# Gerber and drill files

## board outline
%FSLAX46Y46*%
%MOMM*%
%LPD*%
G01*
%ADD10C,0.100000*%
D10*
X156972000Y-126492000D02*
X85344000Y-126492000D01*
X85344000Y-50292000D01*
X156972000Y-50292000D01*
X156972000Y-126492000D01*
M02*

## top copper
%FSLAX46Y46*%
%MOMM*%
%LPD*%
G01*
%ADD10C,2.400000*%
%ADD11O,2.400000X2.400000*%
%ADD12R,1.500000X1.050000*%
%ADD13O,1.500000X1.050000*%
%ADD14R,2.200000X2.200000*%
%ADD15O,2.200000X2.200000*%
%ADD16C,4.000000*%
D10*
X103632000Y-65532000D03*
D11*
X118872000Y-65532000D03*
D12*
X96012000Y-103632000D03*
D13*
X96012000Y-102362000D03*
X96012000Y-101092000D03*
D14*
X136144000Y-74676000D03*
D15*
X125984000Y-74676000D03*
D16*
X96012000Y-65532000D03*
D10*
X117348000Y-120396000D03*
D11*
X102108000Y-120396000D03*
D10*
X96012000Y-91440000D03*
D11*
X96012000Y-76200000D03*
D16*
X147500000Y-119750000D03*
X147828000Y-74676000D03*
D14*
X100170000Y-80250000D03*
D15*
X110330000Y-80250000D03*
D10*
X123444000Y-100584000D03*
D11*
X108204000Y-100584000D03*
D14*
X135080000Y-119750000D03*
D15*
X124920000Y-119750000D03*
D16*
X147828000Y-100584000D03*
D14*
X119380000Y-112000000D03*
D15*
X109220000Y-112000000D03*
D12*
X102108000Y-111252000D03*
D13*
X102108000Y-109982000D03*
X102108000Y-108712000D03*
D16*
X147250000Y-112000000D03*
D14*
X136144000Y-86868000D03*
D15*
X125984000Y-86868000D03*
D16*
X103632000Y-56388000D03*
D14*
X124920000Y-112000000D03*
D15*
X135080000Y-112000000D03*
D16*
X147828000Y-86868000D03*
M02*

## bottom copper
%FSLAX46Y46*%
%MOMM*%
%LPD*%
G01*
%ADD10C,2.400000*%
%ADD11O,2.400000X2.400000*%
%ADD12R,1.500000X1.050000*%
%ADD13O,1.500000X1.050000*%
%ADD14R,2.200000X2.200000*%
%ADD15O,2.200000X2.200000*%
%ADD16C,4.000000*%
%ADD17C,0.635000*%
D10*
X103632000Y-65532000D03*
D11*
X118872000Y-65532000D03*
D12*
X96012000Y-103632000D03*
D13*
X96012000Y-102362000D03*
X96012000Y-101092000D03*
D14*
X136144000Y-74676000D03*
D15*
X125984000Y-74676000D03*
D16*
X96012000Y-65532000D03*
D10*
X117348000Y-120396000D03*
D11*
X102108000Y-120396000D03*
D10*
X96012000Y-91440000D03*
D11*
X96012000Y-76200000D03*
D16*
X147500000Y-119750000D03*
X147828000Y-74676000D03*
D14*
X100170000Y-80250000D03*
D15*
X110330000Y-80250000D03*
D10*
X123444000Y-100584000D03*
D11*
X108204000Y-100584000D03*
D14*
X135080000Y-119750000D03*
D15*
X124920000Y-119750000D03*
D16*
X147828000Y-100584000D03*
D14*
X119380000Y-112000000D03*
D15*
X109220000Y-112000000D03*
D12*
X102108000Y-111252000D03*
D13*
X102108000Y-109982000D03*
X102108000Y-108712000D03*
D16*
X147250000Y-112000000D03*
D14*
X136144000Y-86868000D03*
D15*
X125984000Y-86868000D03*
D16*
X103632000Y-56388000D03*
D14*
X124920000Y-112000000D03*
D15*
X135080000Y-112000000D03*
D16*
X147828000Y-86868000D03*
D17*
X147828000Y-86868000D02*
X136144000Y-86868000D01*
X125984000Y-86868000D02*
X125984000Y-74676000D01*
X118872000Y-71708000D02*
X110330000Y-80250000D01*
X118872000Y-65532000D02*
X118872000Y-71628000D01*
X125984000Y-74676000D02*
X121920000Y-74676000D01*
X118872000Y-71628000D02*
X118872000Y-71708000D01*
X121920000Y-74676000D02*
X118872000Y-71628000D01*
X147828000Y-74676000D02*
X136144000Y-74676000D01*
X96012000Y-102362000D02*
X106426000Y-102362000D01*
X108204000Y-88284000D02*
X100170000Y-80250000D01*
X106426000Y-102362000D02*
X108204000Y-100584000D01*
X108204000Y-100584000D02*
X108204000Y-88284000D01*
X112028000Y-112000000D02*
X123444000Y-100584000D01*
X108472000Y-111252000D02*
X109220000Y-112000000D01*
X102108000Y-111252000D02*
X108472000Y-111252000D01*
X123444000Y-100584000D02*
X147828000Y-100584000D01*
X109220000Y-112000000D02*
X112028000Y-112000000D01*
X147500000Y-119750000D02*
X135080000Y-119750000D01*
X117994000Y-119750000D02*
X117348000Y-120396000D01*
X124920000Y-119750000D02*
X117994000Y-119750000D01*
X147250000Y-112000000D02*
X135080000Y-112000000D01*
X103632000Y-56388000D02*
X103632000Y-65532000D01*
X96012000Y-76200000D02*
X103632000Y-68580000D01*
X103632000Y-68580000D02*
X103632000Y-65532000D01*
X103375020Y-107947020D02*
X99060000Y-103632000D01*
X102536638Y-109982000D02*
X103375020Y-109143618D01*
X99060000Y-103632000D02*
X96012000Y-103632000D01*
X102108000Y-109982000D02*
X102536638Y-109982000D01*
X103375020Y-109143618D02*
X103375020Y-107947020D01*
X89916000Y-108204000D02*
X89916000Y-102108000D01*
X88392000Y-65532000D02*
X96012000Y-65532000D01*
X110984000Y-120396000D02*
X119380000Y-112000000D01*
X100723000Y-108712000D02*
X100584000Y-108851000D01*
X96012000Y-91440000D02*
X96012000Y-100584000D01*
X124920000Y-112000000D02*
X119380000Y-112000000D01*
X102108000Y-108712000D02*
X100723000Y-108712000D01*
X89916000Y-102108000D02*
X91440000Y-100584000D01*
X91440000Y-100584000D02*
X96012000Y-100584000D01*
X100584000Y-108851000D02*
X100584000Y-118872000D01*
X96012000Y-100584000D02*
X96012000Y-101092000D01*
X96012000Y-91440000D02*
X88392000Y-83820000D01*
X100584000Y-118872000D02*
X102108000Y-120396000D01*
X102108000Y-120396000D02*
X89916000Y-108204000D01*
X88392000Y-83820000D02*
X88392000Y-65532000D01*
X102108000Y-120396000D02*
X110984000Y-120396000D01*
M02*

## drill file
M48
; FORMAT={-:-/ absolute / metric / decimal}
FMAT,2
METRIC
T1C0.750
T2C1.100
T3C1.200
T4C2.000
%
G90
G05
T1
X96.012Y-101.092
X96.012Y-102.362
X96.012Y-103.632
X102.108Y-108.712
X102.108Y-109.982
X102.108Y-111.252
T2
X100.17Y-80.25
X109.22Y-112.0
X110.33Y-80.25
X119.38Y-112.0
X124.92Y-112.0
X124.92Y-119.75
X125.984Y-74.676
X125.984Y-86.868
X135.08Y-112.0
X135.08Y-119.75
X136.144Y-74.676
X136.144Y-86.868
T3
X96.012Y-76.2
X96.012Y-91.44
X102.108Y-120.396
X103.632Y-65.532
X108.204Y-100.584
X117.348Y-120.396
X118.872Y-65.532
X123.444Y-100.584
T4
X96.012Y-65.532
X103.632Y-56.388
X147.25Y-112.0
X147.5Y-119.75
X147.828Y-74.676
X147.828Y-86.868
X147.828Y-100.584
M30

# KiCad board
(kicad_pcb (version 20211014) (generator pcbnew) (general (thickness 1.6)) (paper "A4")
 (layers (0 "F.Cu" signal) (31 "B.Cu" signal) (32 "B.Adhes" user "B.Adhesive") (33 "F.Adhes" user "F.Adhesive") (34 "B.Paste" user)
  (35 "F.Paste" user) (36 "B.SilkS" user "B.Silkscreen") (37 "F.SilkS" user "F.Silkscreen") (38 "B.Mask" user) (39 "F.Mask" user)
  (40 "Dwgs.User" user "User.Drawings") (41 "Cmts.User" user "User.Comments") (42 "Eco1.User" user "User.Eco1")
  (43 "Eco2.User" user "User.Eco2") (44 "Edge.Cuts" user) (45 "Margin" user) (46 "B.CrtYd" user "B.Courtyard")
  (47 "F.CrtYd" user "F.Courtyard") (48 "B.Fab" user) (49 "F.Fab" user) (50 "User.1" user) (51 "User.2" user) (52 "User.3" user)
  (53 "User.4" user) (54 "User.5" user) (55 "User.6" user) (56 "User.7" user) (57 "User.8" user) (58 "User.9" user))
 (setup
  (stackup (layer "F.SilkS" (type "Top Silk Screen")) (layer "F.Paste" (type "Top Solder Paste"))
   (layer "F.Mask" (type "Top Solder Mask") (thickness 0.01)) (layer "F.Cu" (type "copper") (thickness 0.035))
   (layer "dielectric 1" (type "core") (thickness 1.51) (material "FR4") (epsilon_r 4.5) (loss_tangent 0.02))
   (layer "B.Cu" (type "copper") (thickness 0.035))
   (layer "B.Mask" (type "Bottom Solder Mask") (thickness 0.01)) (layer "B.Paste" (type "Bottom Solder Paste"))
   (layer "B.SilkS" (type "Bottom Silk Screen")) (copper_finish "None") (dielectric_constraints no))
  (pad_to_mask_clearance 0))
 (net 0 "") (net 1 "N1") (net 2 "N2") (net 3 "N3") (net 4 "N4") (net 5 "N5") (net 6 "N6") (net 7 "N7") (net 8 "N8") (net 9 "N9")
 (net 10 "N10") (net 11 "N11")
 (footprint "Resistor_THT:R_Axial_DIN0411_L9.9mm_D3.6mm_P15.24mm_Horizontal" (layer "F.Cu") (at 103.632 65.532)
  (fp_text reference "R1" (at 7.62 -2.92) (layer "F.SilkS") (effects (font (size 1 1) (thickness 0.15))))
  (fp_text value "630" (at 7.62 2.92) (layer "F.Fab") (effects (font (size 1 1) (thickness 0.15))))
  (pad "1" thru_hole circle (at 0 0) (size 2.4 2.4) (drill 1.2) (layers *.Cu *.Mask) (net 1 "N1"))
  (pad "2" thru_hole oval (at 15.24 0) (size 2.4 2.4) (drill 1.2) (layers *.Cu *.Mask) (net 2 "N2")))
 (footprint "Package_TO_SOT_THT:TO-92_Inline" (layer "F.Cu") (at 96.012 103.632 90)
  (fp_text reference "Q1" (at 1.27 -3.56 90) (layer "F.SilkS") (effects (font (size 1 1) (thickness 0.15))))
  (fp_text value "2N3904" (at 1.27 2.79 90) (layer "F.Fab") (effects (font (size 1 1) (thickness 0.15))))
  (pad "1" thru_hole rect (at 0 0 90) (size 1.05 1.5) (drill 0.75) (layers *.Cu *.Mask) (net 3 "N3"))
  (pad "2" thru_hole oval (at 1.27 0 90) (size 1.05 1.5) (drill 0.75) (layers *.Cu *.Mask) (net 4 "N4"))
  (pad "3" thru_hole oval (at 2.54 0 90) (size 1.05 1.5) (drill 0.75) (layers *.Cu *.Mask) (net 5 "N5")))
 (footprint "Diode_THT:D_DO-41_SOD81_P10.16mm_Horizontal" (layer "F.Cu") (at 136.144 74.676 180)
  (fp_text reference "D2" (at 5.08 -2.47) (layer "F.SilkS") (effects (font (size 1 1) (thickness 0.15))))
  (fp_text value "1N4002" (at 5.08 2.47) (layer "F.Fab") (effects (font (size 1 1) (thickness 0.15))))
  (pad "1" thru_hole rect (at 0 0 180) (size 2.2 2.2) (drill 1.1) (layers *.Cu *.Mask) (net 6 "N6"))
  (pad "2" thru_hole oval (at 10.16 0 180) (size 2.2 2.2) (drill 1.1) (layers *.Cu *.Mask) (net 2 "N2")))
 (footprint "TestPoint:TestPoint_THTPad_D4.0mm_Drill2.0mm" (layer "F.Cu") (at 96.012 65.532)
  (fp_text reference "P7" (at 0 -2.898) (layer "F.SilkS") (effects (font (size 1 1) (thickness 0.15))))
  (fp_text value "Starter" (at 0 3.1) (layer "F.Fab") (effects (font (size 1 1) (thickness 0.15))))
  (pad "1" thru_hole circle (at 0 0) (size 4 4) (drill 2) (layers *.Cu *.Mask) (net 5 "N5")))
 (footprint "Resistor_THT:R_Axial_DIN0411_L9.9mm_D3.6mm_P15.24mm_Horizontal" (layer "F.Cu") (at 117.348 120.396 180)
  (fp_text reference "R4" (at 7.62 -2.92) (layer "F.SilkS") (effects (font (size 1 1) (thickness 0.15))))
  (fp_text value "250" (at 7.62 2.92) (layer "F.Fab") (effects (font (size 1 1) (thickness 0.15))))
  (pad "1" thru_hole circle (at 0 0 180) (size 2.4 2.4) (drill 1.2) (layers *.Cu *.Mask) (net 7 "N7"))
  (pad "2" thru_hole oval (at 15.24 0 180) (size 2.4 2.4) (drill 1.2) (layers *.Cu *.Mask) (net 5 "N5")))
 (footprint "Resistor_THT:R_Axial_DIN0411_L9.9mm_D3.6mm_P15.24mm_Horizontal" (layer "F.Cu") (at 96.012 91.44 90)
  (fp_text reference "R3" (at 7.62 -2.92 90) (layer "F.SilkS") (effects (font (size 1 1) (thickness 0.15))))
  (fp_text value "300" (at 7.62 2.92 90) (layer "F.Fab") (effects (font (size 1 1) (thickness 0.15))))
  (pad "1" thru_hole circle (at 0 0 90) (size 2.4 2.4) (drill 1.2) (layers *.Cu *.Mask) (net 5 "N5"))
  (pad "2" thru_hole oval (at 15.24 0 90) (size 2.4 2.4) (drill 1.2) (layers *.Cu *.Mask) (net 1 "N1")))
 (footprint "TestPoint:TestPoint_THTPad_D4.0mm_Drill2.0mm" (layer "F.Cu") (at 147.5 119.75)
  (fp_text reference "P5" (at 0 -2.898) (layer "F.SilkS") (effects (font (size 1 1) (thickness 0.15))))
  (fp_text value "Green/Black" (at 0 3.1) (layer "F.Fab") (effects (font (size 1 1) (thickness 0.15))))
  (pad "1" thru_hole circle (at 0 0) (size 4 4) (drill 2) (layers *.Cu *.Mask) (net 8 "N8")))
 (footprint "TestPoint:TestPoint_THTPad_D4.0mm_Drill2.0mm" (layer "F.Cu") (at 147.828 74.676)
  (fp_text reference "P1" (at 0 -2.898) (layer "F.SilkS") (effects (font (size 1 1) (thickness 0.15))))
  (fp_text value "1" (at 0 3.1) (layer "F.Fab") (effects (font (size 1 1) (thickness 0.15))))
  (pad "1" thru_hole circle (at 0 0) (size 4 4) (drill 2) (layers *.Cu *.Mask) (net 6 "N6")))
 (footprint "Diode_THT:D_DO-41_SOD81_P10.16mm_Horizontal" (layer "F.Cu") (at 100.17 80.25)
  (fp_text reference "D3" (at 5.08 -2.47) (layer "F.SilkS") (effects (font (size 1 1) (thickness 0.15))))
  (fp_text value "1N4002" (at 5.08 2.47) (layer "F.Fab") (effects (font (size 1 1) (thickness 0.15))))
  (pad "1" thru_hole rect (at 0 0) (size 2.2 2.2) (drill 1.1) (layers *.Cu *.Mask) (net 4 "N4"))
  (pad "2" thru_hole oval (at 10.16 0) (size 2.2 2.2) (drill 1.1) (layers *.Cu *.Mask) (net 2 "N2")))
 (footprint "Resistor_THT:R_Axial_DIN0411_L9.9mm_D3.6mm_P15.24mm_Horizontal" (layer "F.Cu") (at 123.444 100.584 180)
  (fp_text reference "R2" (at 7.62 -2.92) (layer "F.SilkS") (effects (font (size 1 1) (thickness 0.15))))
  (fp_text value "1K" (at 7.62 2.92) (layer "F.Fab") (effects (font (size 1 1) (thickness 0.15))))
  (pad "1" thru_hole circle (at 0 0 180) (size 2.4 2.4) (drill 1.2) (layers *.Cu *.Mask) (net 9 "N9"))
  (pad "2" thru_hole oval (at 15.24 0 180) (size 2.4 2.4) (drill 1.2) (layers *.Cu *.Mask) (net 4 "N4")))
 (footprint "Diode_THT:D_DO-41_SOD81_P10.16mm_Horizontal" (layer "F.Cu") (at 135.08 119.75 180)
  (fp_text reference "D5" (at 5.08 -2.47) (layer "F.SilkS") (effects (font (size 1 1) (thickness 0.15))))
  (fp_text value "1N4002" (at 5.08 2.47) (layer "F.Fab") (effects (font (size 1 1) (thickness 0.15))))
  (pad "1" thru_hole rect (at 0 0 180) (size 2.2 2.2) (drill 1.1) (layers *.Cu *.Mask) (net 8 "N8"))
  (pad "2" thru_hole oval (at 10.16 0 180) (size 2.2 2.2) (drill 1.1) (layers *.Cu *.Mask) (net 7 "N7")))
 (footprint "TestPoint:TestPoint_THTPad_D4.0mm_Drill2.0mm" (layer "F.Cu") (at 147.828 100.584)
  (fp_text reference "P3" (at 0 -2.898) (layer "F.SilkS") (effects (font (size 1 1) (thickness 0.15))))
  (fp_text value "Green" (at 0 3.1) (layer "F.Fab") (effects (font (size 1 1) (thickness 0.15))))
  (pad "1" thru_hole circle (at 0 0) (size 4 4) (drill 2) (layers *.Cu *.Mask) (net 9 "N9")))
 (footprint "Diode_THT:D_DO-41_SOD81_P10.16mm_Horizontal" (layer "F.Cu") (at 119.38 112 180)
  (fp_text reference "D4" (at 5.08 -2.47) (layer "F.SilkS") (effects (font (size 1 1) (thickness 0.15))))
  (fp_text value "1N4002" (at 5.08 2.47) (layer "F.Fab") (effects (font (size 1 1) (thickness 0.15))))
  (pad "1" thru_hole rect (at 0 0 180) (size 2.2 2.2) (drill 1.1) (layers *.Cu *.Mask) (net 5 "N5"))
  (pad "2" thru_hole oval (at 10.16 0 180) (size 2.2 2.2) (drill 1.1) (layers *.Cu *.Mask) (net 9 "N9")))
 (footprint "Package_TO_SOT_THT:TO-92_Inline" (layer "F.Cu") (at 102.108 111.252 90)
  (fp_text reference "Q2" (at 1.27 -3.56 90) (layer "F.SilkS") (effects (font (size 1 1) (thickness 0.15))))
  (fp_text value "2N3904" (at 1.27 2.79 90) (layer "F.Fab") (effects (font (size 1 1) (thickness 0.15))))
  (pad "1" thru_hole rect (at 0 0 90) (size 1.05 1.5) (drill 0.75) (layers *.Cu *.Mask) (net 9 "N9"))
  (pad "2" thru_hole oval (at 1.27 0 90) (size 1.05 1.5) (drill 0.75) (layers *.Cu *.Mask) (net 3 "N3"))
  (pad "3" thru_hole oval (at 2.54 0 90) (size 1.05 1.5) (drill 0.75) (layers *.Cu *.Mask) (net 5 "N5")))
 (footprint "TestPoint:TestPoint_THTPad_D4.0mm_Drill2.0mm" (layer "F.Cu") (at 147.25 112)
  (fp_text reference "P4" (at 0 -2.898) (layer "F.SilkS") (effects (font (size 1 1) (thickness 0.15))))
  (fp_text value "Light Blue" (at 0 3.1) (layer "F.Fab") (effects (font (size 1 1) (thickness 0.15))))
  (pad "1" thru_hole circle (at 0 0) (size 4 4) (drill 2) (layers *.Cu *.Mask) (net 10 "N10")))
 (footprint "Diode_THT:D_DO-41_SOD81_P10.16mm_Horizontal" (layer "F.Cu") (at 136.144 86.868 180)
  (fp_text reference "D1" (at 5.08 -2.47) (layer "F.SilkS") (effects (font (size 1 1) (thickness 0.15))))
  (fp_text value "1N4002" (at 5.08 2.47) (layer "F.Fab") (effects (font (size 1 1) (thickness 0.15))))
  (pad "1" thru_hole rect (at 0 0 180) (size 2.2 2.2) (drill 1.1) (layers *.Cu *.Mask) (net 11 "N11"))
  (pad "2" thru_hole oval (at 10.16 0 180) (size 2.2 2.2) (drill 1.1) (layers *.Cu *.Mask) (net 2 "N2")))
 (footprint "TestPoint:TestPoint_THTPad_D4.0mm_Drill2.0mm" (layer "F.Cu") (at 103.632 56.388)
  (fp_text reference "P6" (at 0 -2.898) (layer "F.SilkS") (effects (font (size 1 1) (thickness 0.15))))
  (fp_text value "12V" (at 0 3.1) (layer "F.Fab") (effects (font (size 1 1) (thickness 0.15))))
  (pad "1" thru_hole circle (at 0 0) (size 4 4) (drill 2) (layers *.Cu *.Mask) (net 1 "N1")))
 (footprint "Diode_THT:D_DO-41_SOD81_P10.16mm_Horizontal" (layer "F.Cu") (at 124.92 112)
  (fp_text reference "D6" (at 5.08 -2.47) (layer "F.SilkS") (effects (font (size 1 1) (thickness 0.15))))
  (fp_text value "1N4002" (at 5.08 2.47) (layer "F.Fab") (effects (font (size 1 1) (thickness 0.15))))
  (pad "1" thru_hole rect (at 0 0) (size 2.2 2.2) (drill 1.1) (layers *.Cu *.Mask) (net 5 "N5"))
  (pad "2" thru_hole oval (at 10.16 0) (size 2.2 2.2) (drill 1.1) (layers *.Cu *.Mask) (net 10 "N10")))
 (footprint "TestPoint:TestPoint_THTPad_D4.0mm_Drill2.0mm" (layer "F.Cu") (at 147.828 86.868)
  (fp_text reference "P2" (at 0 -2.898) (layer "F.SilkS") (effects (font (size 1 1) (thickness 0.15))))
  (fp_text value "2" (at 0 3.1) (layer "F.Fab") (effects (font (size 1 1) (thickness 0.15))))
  (pad "1" thru_hole circle (at 0 0) (size 4 4) (drill 2) (layers *.Cu *.Mask) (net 11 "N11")))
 (gr_poly (pts (xy 156.972 126.492) (xy 85.344 126.492) (xy 85.344 50.292) (xy 156.972 50.292)) (layer "Edge.Cuts") (width 0.1) (fill none))
 (segment (start 147.828 86.868) (end 136.144 86.868) (width 0.635) (layer "B.Cu") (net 11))
 (segment (start 125.984 86.868) (end 125.984 74.676) (width 0.635) (layer "B.Cu") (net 2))
 (segment (start 118.872 71.708) (end 110.33 80.25) (width 0.635) (layer "B.Cu") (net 2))
 (segment (start 118.872 65.532) (end 118.872 71.628) (width 0.635) (layer "B.Cu") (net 2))
 (segment (start 125.984 74.676) (end 121.92 74.676) (width 0.635) (layer "B.Cu") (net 2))
 (segment (start 118.872 71.628) (end 118.872 71.708) (width 0.635) (layer "B.Cu") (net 2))
 (segment (start 121.92 74.676) (end 118.872 71.628) (width 0.635) (layer "B.Cu") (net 2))
 (segment (start 147.828 74.676) (end 136.144 74.676) (width 0.635) (layer "B.Cu") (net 6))
 (segment (start 96.012 102.362) (end 106.426 102.362) (width 0.635) (layer "B.Cu") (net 4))
 (segment (start 108.204 88.284) (end 100.17 80.25) (width 0.635) (layer "B.Cu") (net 4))
 (segment (start 106.426 102.362) (end 108.204 100.584) (width 0.635) (layer "B.Cu") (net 4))
 (segment (start 108.204 100.584) (end 108.204 88.284) (width 0.635) (layer "B.Cu") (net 4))
 (segment (start 112.028 112) (end 123.444 100.584) (width 0.635) (layer "B.Cu") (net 9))
 (segment (start 108.472 111.252) (end 109.22 112) (width 0.635) (layer "B.Cu") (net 9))
 (segment (start 102.108 111.252) (end 108.472 111.252) (width 0.635) (layer "B.Cu") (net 9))
 (segment (start 123.444 100.584) (end 147.828 100.584) (width 0.635) (layer "B.Cu") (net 9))
 (segment (start 109.22 112) (end 112.028 112) (width 0.635) (layer "B.Cu") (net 9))
 (segment (start 147.5 119.75) (end 135.08 119.75) (width 0.635) (layer "B.Cu") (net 8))
 (segment (start 117.994 119.75) (end 117.348 120.396) (width 0.635) (layer "B.Cu") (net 7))
 (segment (start 124.92 119.75) (end 117.994 119.75) (width 0.635) (layer "B.Cu") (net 7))
 (segment (start 147.25 112) (end 135.08 112) (width 0.635) (layer "B.Cu") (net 10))
 (segment (start 103.632 56.388) (end 103.632 65.532) (width 0.635) (layer "B.Cu") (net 1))
 (segment (start 96.012 76.2) (end 103.632 68.58) (width 0.635) (layer "B.Cu") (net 1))
 (segment (start 103.632 68.58) (end 103.632 65.532) (width 0.635) (layer "B.Cu") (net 1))
 (segment (start 103.37502 107.94702) (end 99.06 103.632) (width 0.635) (layer "B.Cu") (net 3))
 (segment (start 102.536638 109.982) (end 103.37502 109.143618) (width 0.635) (layer "B.Cu") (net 3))
 (segment (start 99.06 103.632) (end 96.012 103.632) (width 0.635) (layer "B.Cu") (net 3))
 (segment (start 102.108 109.982) (end 102.536638 109.982) (width 0.635) (layer "B.Cu") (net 3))
 (segment (start 103.37502 109.143618) (end 103.37502 107.94702) (width 0.635) (layer "B.Cu") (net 3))
 (segment (start 89.916 108.204) (end 89.916 102.108) (width 0.635) (layer "B.Cu") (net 5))
 (segment (start 88.392 65.532) (end 96.012 65.532) (width 0.635) (layer "B.Cu") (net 5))
 (segment (start 110.984 120.396) (end 119.38 112) (width 0.635) (layer "B.Cu") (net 5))
 (segment (start 100.723 108.712) (end 100.584 108.851) (width 0.635) (layer "B.Cu") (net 5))
 (segment (start 96.012 91.44) (end 96.012 100.584) (width 0.635) (layer "B.Cu") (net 5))
 (segment (start 124.92 112) (end 119.38 112) (width 0.635) (layer "B.Cu") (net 5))
 (segment (start 102.108 108.712) (end 100.723 108.712) (width 0.635) (layer "B.Cu") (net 5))
 (segment (start 89.916 102.108) (end 91.44 100.584) (width 0.635) (layer "B.Cu") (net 5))
 (segment (start 91.44 100.584) (end 96.012 100.584) (width 0.635) (layer "B.Cu") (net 5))
 (segment (start 100.584 108.851) (end 100.584 118.872) (width 0.635) (layer "B.Cu") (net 5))
 (segment (start 96.012 100.584) (end 96.012 101.092) (width 0.635) (layer "B.Cu") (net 5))
 (segment (start 96.012 91.44) (end 88.392 83.82) (width 0.635) (layer "B.Cu") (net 5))
 (segment (start 100.584 118.872) (end 102.108 120.396) (width 0.635) (layer "B.Cu") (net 5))
 (segment (start 102.108 120.396) (end 89.916 108.204) (width 0.635) (layer "B.Cu") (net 5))
 (segment (start 88.392 83.82) (end 88.392 65.532) (width 0.635) (layer "B.Cu") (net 5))
 (segment (start 102.108 120.396) (end 110.984 120.396) (width 0.635) (layer "B.Cu") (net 5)))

